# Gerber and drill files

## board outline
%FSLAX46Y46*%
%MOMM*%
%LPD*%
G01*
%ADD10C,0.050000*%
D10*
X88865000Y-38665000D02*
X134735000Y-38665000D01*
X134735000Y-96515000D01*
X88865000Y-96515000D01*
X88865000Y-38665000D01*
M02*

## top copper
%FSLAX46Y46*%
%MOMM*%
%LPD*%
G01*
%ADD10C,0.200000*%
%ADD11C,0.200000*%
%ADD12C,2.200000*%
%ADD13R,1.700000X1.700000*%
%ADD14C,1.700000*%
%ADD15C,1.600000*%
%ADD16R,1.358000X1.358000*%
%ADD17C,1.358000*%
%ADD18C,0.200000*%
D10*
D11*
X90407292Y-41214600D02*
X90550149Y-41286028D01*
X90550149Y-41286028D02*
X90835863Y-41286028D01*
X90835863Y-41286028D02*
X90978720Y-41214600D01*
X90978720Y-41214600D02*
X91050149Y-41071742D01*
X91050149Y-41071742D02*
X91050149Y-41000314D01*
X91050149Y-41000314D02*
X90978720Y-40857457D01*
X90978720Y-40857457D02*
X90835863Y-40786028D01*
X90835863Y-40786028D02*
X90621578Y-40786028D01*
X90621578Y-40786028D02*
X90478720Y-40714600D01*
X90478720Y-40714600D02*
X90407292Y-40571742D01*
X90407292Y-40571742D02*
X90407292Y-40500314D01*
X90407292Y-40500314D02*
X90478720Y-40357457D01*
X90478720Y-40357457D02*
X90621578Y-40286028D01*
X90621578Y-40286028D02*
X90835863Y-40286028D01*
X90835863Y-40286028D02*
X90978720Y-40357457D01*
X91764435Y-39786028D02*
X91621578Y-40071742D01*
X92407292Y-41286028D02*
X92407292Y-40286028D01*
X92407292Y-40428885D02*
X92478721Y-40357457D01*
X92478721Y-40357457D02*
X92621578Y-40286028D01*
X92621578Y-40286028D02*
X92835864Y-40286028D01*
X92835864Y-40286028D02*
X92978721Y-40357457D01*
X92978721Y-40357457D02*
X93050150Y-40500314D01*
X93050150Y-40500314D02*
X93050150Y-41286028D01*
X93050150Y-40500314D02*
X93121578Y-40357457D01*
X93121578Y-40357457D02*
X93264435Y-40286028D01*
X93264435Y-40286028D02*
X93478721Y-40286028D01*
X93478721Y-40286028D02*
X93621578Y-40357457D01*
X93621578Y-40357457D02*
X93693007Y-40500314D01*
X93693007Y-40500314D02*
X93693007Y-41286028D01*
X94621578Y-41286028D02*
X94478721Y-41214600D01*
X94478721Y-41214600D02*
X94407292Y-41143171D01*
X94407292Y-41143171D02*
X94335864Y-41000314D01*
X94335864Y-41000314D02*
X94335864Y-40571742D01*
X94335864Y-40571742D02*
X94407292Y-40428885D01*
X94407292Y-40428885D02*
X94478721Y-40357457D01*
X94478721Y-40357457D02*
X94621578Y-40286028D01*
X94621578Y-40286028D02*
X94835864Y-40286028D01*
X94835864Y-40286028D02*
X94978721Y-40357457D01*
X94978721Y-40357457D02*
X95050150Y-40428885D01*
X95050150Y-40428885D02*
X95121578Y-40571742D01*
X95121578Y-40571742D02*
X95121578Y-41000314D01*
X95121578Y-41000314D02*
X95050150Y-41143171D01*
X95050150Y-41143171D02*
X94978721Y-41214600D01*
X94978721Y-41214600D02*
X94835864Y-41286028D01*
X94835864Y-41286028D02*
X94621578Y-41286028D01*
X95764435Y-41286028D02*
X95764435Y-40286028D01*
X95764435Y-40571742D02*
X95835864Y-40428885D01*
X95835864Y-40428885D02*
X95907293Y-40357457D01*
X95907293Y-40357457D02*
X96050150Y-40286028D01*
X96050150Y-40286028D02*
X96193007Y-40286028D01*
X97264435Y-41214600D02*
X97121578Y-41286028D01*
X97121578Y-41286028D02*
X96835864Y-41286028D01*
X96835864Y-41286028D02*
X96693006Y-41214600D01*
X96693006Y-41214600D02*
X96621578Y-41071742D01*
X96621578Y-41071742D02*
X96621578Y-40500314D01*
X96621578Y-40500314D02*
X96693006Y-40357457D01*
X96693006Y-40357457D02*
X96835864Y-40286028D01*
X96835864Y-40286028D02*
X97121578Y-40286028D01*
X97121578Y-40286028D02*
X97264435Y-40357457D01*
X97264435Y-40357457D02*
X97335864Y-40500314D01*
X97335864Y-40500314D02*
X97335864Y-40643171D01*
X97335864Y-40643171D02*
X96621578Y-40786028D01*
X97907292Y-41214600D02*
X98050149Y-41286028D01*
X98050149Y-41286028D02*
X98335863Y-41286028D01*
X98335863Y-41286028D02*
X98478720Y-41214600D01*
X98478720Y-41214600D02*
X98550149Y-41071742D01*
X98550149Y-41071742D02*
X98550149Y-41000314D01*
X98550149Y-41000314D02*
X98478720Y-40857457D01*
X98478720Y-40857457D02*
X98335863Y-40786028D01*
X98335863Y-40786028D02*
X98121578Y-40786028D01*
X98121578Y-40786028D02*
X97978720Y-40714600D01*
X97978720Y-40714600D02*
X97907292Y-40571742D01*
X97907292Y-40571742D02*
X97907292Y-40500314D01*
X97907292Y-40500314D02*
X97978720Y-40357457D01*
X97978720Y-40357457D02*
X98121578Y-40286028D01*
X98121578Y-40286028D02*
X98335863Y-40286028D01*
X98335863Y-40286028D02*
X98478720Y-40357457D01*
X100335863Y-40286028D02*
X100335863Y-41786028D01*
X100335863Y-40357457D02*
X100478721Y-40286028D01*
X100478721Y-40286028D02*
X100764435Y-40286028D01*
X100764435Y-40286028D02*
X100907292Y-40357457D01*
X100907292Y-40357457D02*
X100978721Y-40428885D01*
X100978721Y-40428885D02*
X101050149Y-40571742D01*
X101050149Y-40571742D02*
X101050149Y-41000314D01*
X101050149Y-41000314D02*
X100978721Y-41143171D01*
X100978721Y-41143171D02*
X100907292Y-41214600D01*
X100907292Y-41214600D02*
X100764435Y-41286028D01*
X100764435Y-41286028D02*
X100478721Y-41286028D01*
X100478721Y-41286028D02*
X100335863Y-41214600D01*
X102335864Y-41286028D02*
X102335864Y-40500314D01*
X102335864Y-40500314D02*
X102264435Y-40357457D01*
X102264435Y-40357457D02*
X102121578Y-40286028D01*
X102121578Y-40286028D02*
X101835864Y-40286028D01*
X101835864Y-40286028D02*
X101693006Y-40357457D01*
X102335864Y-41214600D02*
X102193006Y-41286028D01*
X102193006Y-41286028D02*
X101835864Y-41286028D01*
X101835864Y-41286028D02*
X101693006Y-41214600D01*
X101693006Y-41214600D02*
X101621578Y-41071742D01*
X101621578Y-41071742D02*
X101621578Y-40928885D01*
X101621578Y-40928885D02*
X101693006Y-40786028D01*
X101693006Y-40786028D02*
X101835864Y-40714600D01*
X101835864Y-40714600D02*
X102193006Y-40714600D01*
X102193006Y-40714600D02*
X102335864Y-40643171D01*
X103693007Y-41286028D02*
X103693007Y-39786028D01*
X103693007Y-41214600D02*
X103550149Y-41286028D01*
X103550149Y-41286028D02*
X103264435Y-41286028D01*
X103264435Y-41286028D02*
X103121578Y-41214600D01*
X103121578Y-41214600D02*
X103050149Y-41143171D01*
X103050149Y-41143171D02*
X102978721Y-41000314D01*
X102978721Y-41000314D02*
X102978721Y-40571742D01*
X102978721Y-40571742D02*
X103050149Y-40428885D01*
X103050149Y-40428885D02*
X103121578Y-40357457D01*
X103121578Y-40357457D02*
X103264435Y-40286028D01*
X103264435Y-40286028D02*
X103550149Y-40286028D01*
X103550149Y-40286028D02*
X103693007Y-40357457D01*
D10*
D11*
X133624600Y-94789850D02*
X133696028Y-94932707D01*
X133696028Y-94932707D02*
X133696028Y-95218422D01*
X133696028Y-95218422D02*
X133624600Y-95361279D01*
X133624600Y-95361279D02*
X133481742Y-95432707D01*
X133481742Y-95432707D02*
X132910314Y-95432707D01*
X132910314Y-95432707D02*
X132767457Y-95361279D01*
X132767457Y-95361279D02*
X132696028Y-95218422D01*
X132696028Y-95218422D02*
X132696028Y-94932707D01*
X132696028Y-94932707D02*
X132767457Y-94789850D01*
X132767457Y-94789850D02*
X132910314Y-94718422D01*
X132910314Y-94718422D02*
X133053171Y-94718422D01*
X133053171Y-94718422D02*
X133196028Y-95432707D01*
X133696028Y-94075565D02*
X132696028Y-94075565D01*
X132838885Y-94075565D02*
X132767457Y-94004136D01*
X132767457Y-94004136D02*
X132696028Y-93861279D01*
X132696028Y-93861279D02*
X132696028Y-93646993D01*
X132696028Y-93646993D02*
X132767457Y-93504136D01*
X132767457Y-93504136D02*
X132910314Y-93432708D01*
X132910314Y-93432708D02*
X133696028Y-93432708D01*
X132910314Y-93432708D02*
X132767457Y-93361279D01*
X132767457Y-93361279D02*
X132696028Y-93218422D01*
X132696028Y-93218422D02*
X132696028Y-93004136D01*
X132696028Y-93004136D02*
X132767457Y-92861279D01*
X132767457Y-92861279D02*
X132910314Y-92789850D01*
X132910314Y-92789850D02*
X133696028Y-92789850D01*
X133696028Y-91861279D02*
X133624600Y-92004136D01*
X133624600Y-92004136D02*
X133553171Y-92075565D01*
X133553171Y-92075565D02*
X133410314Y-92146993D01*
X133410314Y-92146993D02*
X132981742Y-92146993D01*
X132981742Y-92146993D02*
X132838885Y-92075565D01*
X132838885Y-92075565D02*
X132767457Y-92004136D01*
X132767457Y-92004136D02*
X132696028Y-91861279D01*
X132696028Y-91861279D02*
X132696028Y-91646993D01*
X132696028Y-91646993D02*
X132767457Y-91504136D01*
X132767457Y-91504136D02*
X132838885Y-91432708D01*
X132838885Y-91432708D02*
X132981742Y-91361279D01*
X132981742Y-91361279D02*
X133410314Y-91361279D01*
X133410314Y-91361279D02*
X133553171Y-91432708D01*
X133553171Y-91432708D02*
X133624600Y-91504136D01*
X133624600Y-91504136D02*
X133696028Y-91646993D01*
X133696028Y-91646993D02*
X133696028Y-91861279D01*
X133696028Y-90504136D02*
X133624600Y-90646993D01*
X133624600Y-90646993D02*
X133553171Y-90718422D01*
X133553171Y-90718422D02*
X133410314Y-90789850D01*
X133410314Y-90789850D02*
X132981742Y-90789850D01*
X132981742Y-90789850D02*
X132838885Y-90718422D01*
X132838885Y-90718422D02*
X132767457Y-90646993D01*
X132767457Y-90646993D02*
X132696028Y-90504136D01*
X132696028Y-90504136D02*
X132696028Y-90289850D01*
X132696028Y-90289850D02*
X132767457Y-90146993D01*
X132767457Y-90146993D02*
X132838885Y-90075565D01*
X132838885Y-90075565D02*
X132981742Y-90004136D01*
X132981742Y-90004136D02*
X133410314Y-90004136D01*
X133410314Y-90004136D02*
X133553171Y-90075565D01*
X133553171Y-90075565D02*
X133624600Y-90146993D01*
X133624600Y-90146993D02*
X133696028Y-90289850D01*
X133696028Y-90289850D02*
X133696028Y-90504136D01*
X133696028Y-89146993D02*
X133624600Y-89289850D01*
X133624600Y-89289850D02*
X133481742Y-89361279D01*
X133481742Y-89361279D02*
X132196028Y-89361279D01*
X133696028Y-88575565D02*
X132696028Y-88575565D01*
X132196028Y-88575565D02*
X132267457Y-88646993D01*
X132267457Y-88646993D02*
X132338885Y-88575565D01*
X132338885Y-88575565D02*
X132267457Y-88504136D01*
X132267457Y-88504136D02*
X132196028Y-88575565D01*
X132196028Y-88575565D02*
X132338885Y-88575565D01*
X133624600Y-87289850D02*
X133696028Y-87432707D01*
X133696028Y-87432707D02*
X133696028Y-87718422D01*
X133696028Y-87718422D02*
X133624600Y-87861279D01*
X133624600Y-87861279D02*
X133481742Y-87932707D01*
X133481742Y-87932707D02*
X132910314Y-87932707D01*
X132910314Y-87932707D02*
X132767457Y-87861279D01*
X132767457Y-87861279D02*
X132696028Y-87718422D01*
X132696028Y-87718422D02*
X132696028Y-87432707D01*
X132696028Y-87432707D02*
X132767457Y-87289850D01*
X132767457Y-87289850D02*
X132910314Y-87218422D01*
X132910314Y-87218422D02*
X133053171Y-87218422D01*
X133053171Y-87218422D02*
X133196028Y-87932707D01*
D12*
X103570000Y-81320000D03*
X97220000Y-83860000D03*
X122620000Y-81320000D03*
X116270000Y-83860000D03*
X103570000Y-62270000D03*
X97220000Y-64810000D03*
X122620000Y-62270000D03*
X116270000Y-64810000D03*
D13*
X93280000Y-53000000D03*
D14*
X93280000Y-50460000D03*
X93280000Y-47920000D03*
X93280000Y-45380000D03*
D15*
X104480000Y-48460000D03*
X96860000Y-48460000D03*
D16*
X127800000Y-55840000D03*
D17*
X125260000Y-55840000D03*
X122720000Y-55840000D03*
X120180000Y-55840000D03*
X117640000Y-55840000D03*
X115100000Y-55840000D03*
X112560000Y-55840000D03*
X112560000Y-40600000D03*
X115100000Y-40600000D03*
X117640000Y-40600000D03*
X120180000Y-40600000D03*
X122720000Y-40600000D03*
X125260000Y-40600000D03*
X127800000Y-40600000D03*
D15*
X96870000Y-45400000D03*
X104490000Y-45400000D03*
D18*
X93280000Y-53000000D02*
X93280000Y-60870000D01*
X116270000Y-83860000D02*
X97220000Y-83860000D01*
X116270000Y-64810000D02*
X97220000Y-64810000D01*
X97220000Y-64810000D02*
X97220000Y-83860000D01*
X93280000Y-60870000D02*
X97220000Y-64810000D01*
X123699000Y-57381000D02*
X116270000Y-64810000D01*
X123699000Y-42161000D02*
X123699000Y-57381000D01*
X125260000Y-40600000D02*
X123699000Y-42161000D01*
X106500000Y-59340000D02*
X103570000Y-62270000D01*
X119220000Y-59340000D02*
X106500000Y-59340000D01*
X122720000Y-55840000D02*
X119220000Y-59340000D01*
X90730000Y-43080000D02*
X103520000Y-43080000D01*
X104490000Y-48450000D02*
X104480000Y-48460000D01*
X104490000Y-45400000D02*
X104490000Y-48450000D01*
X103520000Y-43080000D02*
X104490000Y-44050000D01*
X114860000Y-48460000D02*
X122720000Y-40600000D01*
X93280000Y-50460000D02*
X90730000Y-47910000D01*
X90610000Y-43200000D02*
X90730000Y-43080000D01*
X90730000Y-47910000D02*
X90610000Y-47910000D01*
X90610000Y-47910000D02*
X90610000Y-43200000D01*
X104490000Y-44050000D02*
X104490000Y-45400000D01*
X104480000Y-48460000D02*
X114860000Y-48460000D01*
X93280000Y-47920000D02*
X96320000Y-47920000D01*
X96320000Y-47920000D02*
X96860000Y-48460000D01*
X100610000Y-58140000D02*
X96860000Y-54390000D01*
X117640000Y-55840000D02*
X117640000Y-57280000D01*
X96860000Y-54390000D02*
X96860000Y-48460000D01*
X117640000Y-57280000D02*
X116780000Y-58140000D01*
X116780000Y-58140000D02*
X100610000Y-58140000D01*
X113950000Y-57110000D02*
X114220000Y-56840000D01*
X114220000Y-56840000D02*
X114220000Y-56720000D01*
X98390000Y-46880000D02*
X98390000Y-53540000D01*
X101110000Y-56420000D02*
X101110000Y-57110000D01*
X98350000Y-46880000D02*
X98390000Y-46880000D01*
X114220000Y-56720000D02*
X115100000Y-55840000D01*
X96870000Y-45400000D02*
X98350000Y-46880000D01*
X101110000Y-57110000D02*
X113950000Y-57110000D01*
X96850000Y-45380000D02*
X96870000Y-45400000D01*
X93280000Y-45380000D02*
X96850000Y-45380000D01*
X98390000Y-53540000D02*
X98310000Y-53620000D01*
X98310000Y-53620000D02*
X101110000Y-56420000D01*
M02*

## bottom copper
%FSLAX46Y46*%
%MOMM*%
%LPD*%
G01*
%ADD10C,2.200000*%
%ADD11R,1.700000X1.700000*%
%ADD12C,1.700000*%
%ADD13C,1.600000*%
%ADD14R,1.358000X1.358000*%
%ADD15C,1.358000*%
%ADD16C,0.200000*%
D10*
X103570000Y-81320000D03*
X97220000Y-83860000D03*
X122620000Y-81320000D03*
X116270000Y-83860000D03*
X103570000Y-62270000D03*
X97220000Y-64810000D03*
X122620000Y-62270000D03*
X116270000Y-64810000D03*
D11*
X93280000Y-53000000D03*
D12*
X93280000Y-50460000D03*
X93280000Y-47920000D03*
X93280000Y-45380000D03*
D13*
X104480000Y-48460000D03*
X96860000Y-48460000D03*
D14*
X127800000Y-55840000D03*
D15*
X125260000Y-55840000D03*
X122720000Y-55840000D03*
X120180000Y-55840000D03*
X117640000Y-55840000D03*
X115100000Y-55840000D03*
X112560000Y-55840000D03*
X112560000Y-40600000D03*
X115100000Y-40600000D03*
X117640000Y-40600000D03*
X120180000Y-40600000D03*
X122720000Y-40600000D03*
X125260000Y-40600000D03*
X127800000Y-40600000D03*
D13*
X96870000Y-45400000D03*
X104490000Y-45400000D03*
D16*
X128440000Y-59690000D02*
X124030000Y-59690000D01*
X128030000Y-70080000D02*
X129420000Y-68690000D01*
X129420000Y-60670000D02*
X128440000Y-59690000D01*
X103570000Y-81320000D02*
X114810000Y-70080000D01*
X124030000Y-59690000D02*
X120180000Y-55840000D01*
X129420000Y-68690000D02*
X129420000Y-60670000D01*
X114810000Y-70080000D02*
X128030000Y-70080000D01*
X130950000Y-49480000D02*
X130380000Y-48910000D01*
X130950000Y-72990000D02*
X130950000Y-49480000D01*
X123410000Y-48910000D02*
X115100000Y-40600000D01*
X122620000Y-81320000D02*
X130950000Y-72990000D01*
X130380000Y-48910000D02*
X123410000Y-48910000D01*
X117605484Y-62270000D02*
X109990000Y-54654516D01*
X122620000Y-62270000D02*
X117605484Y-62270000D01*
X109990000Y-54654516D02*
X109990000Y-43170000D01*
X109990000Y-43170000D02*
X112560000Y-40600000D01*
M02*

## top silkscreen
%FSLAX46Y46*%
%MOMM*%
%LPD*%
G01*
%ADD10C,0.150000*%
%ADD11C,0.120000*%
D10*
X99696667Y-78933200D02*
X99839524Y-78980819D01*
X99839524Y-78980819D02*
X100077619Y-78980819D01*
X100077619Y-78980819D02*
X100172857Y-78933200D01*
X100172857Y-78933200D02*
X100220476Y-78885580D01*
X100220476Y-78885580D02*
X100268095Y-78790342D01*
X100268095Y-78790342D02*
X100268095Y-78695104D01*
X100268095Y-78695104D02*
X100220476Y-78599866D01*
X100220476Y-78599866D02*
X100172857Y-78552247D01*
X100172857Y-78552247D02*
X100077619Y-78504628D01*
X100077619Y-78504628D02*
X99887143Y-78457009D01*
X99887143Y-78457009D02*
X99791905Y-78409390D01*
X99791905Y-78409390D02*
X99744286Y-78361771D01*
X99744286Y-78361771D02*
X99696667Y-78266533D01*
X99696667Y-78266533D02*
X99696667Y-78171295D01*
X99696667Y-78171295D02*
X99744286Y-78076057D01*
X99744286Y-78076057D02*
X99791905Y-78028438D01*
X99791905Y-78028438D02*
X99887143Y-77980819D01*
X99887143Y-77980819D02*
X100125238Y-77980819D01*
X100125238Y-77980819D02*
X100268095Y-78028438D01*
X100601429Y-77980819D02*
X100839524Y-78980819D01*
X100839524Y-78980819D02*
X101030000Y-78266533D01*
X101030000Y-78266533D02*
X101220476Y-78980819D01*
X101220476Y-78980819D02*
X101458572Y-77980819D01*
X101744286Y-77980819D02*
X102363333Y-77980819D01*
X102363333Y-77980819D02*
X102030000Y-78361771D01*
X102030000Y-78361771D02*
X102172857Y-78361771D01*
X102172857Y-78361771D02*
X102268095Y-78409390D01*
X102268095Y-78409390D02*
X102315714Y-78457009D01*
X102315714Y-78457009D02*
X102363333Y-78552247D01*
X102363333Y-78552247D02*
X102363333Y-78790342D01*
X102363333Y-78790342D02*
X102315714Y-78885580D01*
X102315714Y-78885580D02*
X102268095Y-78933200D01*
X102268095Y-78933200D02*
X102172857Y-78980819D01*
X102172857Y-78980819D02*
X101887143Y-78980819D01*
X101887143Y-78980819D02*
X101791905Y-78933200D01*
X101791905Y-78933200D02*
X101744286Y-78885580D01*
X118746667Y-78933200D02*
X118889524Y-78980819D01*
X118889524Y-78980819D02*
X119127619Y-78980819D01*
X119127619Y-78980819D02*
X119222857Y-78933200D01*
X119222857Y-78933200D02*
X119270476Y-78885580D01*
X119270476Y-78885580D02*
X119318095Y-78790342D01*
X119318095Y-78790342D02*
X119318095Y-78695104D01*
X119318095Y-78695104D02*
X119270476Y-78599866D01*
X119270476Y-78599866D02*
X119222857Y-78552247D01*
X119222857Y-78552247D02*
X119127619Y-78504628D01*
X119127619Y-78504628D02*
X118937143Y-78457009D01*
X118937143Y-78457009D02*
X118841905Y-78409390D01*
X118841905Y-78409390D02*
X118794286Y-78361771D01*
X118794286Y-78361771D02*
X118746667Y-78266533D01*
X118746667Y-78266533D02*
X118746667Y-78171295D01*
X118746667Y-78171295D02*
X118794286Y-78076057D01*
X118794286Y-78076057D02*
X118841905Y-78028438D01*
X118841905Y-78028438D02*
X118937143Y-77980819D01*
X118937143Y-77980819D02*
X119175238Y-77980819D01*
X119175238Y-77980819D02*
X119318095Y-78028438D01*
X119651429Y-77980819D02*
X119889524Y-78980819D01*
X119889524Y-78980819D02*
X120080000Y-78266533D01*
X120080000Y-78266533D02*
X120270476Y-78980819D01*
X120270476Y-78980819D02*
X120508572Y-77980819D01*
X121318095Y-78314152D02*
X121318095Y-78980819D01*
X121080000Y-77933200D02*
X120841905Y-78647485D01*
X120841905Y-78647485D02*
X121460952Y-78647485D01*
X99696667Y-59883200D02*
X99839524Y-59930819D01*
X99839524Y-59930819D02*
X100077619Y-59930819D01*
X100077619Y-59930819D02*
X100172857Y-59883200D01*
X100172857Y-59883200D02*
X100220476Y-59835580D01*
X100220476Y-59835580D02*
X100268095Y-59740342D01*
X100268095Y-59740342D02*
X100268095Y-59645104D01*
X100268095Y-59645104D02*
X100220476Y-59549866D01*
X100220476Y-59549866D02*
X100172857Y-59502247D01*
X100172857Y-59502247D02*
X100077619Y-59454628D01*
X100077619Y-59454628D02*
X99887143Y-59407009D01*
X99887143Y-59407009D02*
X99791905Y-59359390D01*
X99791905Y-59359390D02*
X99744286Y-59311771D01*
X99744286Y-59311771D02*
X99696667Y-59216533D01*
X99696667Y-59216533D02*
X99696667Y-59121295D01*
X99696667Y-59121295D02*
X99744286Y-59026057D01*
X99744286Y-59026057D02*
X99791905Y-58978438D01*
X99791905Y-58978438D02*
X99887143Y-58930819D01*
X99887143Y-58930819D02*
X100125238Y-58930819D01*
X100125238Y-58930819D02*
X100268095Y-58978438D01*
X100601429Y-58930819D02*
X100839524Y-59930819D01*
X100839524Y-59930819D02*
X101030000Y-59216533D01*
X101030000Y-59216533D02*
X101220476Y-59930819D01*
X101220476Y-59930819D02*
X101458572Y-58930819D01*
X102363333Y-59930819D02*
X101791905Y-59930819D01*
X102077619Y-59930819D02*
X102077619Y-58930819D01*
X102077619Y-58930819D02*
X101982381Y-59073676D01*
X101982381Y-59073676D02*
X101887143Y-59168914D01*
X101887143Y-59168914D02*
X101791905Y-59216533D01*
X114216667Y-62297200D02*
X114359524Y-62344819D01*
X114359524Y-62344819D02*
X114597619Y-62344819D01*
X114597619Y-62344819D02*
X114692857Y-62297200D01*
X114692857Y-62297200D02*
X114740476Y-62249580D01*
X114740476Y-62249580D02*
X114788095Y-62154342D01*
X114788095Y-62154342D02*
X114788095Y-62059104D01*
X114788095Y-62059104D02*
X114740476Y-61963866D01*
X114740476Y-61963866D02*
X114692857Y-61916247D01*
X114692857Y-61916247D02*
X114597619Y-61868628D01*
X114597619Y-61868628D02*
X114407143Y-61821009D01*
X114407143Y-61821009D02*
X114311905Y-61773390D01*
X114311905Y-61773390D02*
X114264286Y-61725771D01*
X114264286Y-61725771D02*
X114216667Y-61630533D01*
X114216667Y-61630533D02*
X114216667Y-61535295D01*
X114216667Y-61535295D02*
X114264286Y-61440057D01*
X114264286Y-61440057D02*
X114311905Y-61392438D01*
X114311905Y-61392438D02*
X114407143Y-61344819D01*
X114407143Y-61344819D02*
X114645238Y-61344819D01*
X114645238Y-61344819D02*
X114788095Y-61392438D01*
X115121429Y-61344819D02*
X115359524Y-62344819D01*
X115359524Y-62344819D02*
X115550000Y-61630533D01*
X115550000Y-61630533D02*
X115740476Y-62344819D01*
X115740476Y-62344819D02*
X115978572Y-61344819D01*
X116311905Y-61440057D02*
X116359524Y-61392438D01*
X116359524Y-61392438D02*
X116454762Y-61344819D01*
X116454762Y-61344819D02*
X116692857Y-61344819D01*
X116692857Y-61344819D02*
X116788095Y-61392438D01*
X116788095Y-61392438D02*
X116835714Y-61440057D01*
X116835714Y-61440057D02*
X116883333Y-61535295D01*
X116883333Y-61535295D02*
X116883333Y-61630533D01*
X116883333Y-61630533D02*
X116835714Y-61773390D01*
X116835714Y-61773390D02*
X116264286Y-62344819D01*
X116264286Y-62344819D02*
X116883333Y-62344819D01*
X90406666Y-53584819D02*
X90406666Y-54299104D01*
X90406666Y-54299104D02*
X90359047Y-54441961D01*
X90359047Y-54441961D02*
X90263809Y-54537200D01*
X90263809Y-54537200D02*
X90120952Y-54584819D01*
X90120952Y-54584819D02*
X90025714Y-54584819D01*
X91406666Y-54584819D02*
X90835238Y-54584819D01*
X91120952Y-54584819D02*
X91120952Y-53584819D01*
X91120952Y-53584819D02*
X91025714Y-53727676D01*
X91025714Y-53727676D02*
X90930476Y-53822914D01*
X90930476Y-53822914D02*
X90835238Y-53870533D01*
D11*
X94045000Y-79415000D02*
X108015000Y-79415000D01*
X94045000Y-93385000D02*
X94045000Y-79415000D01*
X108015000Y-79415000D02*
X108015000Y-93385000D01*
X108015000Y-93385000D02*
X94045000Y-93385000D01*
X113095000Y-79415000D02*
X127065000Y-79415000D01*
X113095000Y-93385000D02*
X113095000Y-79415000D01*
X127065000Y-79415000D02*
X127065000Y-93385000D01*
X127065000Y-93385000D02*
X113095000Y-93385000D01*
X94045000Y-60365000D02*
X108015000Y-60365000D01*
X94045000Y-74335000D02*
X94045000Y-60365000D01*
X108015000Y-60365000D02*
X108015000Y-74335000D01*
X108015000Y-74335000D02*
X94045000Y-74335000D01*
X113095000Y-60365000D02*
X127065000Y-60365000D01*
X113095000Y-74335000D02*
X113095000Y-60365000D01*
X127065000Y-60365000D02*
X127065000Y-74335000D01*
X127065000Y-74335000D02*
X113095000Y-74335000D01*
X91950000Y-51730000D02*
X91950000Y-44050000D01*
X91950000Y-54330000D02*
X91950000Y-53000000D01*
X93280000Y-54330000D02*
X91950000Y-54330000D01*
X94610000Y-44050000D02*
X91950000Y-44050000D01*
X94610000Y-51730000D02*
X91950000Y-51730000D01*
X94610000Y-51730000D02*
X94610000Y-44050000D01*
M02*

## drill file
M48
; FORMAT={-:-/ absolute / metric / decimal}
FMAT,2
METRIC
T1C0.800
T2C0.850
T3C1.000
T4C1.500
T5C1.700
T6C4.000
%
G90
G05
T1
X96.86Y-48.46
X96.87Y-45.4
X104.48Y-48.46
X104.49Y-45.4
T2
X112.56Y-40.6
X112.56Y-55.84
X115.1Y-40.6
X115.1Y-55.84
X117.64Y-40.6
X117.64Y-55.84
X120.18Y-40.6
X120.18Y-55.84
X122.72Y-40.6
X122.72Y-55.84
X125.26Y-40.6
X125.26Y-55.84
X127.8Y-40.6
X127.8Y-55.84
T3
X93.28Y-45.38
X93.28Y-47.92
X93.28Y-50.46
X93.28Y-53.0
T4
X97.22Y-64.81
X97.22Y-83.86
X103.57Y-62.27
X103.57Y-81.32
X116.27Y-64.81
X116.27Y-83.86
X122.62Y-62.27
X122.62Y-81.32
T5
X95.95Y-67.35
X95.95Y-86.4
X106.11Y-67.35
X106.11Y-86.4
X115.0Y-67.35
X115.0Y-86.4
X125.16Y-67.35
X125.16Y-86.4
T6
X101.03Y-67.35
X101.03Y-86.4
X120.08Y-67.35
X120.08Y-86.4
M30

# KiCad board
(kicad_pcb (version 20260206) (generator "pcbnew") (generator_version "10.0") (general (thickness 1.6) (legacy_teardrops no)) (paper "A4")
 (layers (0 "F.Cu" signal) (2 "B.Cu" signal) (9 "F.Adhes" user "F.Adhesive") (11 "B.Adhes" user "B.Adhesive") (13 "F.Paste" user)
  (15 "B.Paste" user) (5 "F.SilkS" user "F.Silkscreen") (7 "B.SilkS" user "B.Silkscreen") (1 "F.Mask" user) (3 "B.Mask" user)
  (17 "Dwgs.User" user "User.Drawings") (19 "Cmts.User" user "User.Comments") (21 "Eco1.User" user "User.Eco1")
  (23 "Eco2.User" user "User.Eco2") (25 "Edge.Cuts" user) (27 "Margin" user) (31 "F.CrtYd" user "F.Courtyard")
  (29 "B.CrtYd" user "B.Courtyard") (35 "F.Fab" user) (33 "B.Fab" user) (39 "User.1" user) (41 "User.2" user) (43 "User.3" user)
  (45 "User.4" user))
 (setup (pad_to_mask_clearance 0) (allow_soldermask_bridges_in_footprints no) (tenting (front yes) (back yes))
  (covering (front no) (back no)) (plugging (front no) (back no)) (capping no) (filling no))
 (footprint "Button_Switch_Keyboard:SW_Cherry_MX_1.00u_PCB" (layer "F.Cu") (at 103.57 81.32)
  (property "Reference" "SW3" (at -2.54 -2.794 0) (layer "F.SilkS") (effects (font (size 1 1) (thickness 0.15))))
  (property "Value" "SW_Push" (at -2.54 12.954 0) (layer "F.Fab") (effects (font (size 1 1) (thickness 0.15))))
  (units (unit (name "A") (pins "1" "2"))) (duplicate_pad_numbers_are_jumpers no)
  (fp_line (start -9.525 -1.905) (end 4.445 -1.905) (stroke (width 0.12) (type solid)) (layer "F.SilkS"))
  (fp_line (start -9.525 12.065) (end -9.525 -1.905) (stroke (width 0.12) (type solid)) (layer "F.SilkS"))
  (fp_line (start 4.445 -1.905) (end 4.445 12.065) (stroke (width 0.12) (type solid)) (layer "F.SilkS"))
  (fp_line (start 4.445 12.065) (end -9.525 12.065) (stroke (width 0.12) (type solid)) (layer "F.SilkS"))
  (pad "" np_thru_hole circle (at -7.62 5.08) (size 1.7 1.7) (drill 1.7) (layers "*.Cu" "*.Mask"))
  (pad "" np_thru_hole circle (at -2.54 5.08) (size 4 4) (drill 4) (layers "*.Cu" "*.Mask"))
  (pad "" np_thru_hole circle (at 2.54 5.08) (size 1.7 1.7) (drill 1.7) (layers "*.Cu" "*.Mask"))
  (pad "1" thru_hole circle (at 0 0) (size 2.2 2.2) (drill 1.5) (layers "*.Cu" "*.Mask") (remove_unused_layers no) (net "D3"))
  (pad "2" thru_hole circle (at -6.35 2.54) (size 2.2 2.2) (drill 1.5) (layers "*.Cu" "*.Mask") (remove_unused_layers no) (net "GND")))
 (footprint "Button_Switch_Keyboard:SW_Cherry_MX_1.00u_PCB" (layer "F.Cu") (at 122.62 81.32)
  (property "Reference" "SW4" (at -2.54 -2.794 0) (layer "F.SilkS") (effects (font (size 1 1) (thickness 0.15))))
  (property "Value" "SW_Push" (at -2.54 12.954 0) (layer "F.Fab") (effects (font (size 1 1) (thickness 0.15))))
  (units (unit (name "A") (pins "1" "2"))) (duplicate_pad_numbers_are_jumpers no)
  (fp_line (start -9.525 -1.905) (end 4.445 -1.905) (stroke (width 0.12) (type solid)) (layer "F.SilkS"))
  (fp_line (start -9.525 12.065) (end -9.525 -1.905) (stroke (width 0.12) (type solid)) (layer "F.SilkS"))
  (fp_line (start 4.445 -1.905) (end 4.445 12.065) (stroke (width 0.12) (type solid)) (layer "F.SilkS"))
  (fp_line (start 4.445 12.065) (end -9.525 12.065) (stroke (width 0.12) (type solid)) (layer "F.SilkS"))
  (pad "" np_thru_hole circle (at -7.62 5.08) (size 1.7 1.7) (drill 1.7) (layers "*.Cu" "*.Mask"))
  (pad "" np_thru_hole circle (at -2.54 5.08) (size 4 4) (drill 4) (layers "*.Cu" "*.Mask"))
  (pad "" np_thru_hole circle (at 2.54 5.08) (size 1.7 1.7) (drill 1.7) (layers "*.Cu" "*.Mask"))
  (pad "1" thru_hole circle (at 0 0) (size 2.2 2.2) (drill 1.5) (layers "*.Cu" "*.Mask") (remove_unused_layers no) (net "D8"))
  (pad "2" thru_hole circle (at -6.35 2.54) (size 2.2 2.2) (drill 1.5) (layers "*.Cu" "*.Mask") (remove_unused_layers no) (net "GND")))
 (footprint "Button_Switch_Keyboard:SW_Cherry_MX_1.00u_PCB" (layer "F.Cu") (at 103.57 62.27)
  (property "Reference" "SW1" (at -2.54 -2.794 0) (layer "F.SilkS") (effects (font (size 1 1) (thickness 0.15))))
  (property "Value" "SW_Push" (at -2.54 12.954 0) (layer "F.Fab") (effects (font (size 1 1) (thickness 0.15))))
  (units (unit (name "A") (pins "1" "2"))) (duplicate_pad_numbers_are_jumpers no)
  (fp_line (start -9.525 -1.905) (end 4.445 -1.905) (stroke (width 0.12) (type solid)) (layer "F.SilkS"))
  (fp_line (start -9.525 12.065) (end -9.525 -1.905) (stroke (width 0.12) (type solid)) (layer "F.SilkS"))
  (fp_line (start 4.445 -1.905) (end 4.445 12.065) (stroke (width 0.12) (type solid)) (layer "F.SilkS"))
  (fp_line (start 4.445 12.065) (end -9.525 12.065) (stroke (width 0.12) (type solid)) (layer "F.SilkS"))
  (pad "" np_thru_hole circle (at -7.62 5.08) (size 1.7 1.7) (drill 1.7) (layers "*.Cu" "*.Mask"))
  (pad "" np_thru_hole circle (at -2.54 5.08) (size 4 4) (drill 4) (layers "*.Cu" "*.Mask"))
  (pad "" np_thru_hole circle (at 2.54 5.08) (size 1.7 1.7) (drill 1.7) (layers "*.Cu" "*.Mask"))
  (pad "1" thru_hole circle (at 0 0) (size 2.2 2.2) (drill 1.5) (layers "*.Cu" "*.Mask") (remove_unused_layers no) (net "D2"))
  (pad "2" thru_hole circle (at -6.35 2.54) (size 2.2 2.2) (drill 1.5) (layers "*.Cu" "*.Mask") (remove_unused_layers no) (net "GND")))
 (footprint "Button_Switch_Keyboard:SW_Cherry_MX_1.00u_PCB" (layer "F.Cu") (at 122.62 62.27)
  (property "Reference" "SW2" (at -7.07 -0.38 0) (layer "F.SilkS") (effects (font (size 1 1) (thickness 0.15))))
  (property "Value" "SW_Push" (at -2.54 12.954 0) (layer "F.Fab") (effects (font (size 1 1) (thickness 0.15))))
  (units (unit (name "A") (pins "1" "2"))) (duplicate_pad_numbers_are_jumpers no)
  (fp_line (start -9.525 -1.905) (end 4.445 -1.905) (stroke (width 0.12) (type solid)) (layer "F.SilkS"))
  (fp_line (start -9.525 12.065) (end -9.525 -1.905) (stroke (width 0.12) (type solid)) (layer "F.SilkS"))
  (fp_line (start 4.445 -1.905) (end 4.445 12.065) (stroke (width 0.12) (type solid)) (layer "F.SilkS"))
  (fp_line (start 4.445 12.065) (end -9.525 12.065) (stroke (width 0.12) (type solid)) (layer "F.SilkS"))
  (pad "" np_thru_hole circle (at -7.62 5.08) (size 1.7 1.7) (drill 1.7) (layers "*.Cu" "*.Mask"))
  (pad "" np_thru_hole circle (at -2.54 5.08) (size 4 4) (drill 4) (layers "*.Cu" "*.Mask"))
  (pad "" np_thru_hole circle (at 2.54 5.08) (size 1.7 1.7) (drill 1.7) (layers "*.Cu" "*.Mask"))
  (pad "1" thru_hole circle (at 0 0) (size 2.2 2.2) (drill 1.5) (layers "*.Cu" "*.Mask") (remove_unused_layers no) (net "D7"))
  (pad "2" thru_hole circle (at -6.35 2.54) (size 2.2 2.2) (drill 1.5) (layers "*.Cu" "*.Mask") (remove_unused_layers no) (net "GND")))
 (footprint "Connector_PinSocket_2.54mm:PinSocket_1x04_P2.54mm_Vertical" (layer "F.Cu") (at 93.28 53 180)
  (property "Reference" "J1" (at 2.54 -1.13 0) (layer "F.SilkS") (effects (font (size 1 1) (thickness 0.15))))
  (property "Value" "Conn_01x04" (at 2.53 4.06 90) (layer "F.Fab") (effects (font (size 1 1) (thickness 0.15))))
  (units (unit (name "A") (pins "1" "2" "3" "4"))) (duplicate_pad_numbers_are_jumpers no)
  (fp_line (start 1.33 1.27) (end 1.33 8.95) (stroke (width 0.12) (type solid)) (layer "F.SilkS"))
  (fp_line (start 1.33 -1.33) (end 1.33 0) (stroke (width 0.12) (type solid)) (layer "F.SilkS"))
  (fp_line (start 0 -1.33) (end 1.33 -1.33) (stroke (width 0.12) (type solid)) (layer "F.SilkS"))
  (fp_line (start -1.33 8.95) (end 1.33 8.95) (stroke (width 0.12) (type solid)) (layer "F.SilkS"))
  (fp_line (start -1.33 1.27) (end 1.33 1.27) (stroke (width 0.12) (type solid)) (layer "F.SilkS"))
  (fp_line (start -1.33 1.27) (end -1.33 8.95) (stroke (width 0.12) (type solid)) (layer "F.SilkS"))
  (pad "1" thru_hole rect (at 0 0 180) (size 1.7 1.7) (drill 1) (layers "*.Cu" "*.Mask") (remove_unused_layers no) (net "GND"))
  (pad "2" thru_hole circle (at 0 2.54 180) (size 1.7 1.7) (drill 1) (layers "*.Cu" "*.Mask") (remove_unused_layers no) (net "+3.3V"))
  (pad "3" thru_hole circle (at 0 5.08 180) (size 1.7 1.7) (drill 1) (layers "*.Cu" "*.Mask") (remove_unused_layers no) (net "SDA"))
  (pad "4" thru_hole circle (at 0 7.62 180) (size 1.7 1.7) (drill 1) (layers "*.Cu" "*.Mask") (remove_unused_layers no) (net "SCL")))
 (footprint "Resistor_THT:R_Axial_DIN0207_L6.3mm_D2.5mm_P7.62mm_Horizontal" (layer "B.Cu") (at 104.48 48.46 180)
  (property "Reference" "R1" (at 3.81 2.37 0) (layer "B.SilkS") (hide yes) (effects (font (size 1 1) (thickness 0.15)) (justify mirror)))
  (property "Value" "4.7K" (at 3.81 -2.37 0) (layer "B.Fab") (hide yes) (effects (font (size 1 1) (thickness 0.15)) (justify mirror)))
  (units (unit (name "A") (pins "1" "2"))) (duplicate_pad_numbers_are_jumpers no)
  (pad "1" thru_hole circle (at 0 0 180) (size 1.6 1.6) (drill 0.8) (layers "*.Cu" "*.Mask") (remove_unused_layers no) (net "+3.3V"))
  (pad "2" thru_hole circle (at 7.62 0 180) (size 1.6 1.6) (drill 0.8) (layers "*.Cu" "*.Mask") (remove_unused_layers no) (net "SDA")))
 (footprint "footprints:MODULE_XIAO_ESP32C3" (layer "B.Cu") (at 120.2435 48.22 90)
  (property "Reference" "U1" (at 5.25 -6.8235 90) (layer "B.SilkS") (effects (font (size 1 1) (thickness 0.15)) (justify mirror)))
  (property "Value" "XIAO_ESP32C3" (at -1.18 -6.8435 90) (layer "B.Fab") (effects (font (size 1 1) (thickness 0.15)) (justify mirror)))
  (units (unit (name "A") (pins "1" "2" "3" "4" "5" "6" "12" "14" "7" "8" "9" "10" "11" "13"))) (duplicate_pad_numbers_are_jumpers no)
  (pad "1" thru_hole rect (at -7.62 7.5565 90) (size 1.358 1.358) (drill 0.85) (layers "*.Cu" "*.Mask") (remove_unused_layers no)
   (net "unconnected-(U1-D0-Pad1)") (solder_mask_margin 0.102))
  (pad "2" thru_hole circle (at -7.62 5.0165 90) (size 1.358 1.358) (drill 0.85) (layers "*.Cu" "*.Mask") (remove_unused_layers no)
   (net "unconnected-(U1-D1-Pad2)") (solder_mask_margin 0.102))
  (pad "3" thru_hole circle (at -7.62 2.4765 90) (size 1.358 1.358) (drill 0.85) (layers "*.Cu" "*.Mask") (remove_unused_layers no)
   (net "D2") (solder_mask_margin 0.102))
  (pad "4" thru_hole circle (at -7.62 -0.0635 90) (size 1.358 1.358) (drill 0.85) (layers "*.Cu" "*.Mask") (remove_unused_layers no)
   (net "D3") (solder_mask_margin 0.102))
  (pad "5" thru_hole circle (at -7.62 -2.6035 90) (size 1.358 1.358) (drill 0.85) (layers "*.Cu" "*.Mask") (remove_unused_layers no)
   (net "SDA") (solder_mask_margin 0.102))
  (pad "6" thru_hole circle (at -7.62 -5.1435 90) (size 1.358 1.358) (drill 0.85) (layers "*.Cu" "*.Mask") (remove_unused_layers no)
   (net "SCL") (solder_mask_margin 0.102))
  (pad "7" thru_hole circle (at -7.62 -7.6835 90) (size 1.358 1.358) (drill 0.85) (layers "*.Cu" "*.Mask") (remove_unused_layers no)
   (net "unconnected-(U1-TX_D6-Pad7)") (solder_mask_margin 0.102))
  (pad "8" thru_hole circle (at 7.62 -7.6835 90) (size 1.358 1.358) (drill 0.85) (layers "*.Cu" "*.Mask") (remove_unused_layers no)
   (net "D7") (solder_mask_margin 0.102))
  (pad "9" thru_hole circle (at 7.62 -5.1435 90) (size 1.358 1.358) (drill 0.85) (layers "*.Cu" "*.Mask") (remove_unused_layers no)
   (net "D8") (solder_mask_margin 0.102))
  (pad "10" thru_hole circle (at 7.62 -2.6035 90) (size 1.358 1.358) (drill 0.85) (layers "*.Cu" "*.Mask") (remove_unused_layers no)
   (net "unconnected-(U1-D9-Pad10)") (solder_mask_margin 0.102))
  (pad "11" thru_hole circle (at 7.62 -0.0635 90) (size 1.358 1.358) (drill 0.85) (layers "*.Cu" "*.Mask") (remove_unused_layers no)
   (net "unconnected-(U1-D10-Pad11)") (solder_mask_margin 0.102))
  (pad "12" thru_hole circle (at 7.62 2.4765 90) (size 1.358 1.358) (drill 0.85) (layers "*.Cu" "*.Mask") (remove_unused_layers no)
   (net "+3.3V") (solder_mask_margin 0.102))
  (pad "13" thru_hole circle (at 7.62 5.0165 90) (size 1.358 1.358) (drill 0.85) (layers "*.Cu" "*.Mask") (remove_unused_layers no)
   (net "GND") (solder_mask_margin 0.102))
  (pad "14" thru_hole circle (at 7.62 7.5565 90) (size 1.358 1.358) (drill 0.85) (layers "*.Cu" "*.Mask") (remove_unused_layers no)
   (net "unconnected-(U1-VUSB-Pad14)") (solder_mask_margin 0.102)))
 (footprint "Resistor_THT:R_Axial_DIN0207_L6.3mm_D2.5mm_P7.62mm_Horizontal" (layer "B.Cu") (at 96.87 45.4)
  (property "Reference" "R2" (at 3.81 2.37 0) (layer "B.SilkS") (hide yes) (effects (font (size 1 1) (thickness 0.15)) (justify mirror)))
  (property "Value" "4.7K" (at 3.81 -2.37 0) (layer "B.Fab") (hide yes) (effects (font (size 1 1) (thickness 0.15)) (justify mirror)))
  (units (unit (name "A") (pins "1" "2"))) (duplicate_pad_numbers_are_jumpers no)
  (pad "1" thru_hole circle (at 0 0) (size 1.6 1.6) (drill 0.8) (layers "*.Cu" "*.Mask") (remove_unused_layers no) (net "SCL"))
  (pad "2" thru_hole circle (at 7.62 0) (size 1.6 1.6) (drill 0.8) (layers "*.Cu" "*.Mask") (remove_unused_layers no) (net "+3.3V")))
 (gr_rect (start 88.865 38.665) (end 134.735 96.515) (stroke (width 0.05) (type default)) (fill no) (layer "Edge.Cuts"))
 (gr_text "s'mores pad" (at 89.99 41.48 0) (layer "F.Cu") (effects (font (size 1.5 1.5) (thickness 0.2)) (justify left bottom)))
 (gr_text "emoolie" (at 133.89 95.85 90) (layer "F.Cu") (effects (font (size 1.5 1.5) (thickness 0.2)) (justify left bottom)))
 (segment (start 128.44 59.69) (end 124.03 59.69) (width 0.2) (layer "B.Cu") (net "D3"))
 (segment (start 128.03 70.08) (end 129.42 68.69) (width 0.2) (layer "B.Cu") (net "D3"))
 (segment (start 129.42 60.67) (end 128.44 59.69) (width 0.2) (layer "B.Cu") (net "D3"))
 (segment (start 103.57 81.32) (end 114.81 70.08) (width 0.2) (layer "B.Cu") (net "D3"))
 (segment (start 124.03 59.69) (end 120.18 55.84) (width 0.2) (layer "B.Cu") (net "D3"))
 (segment (start 129.42 68.69) (end 129.42 60.67) (width 0.2) (layer "B.Cu") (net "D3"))
 (segment (start 114.81 70.08) (end 128.03 70.08) (width 0.2) (layer "B.Cu") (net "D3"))
 (segment (start 93.28 53) (end 93.28 60.87) (width 0.2) (layer "F.Cu") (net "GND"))
 (segment (start 116.27 83.86) (end 97.22 83.86) (width 0.2) (layer "F.Cu") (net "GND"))
 (segment (start 116.27 64.81) (end 97.22 64.81) (width 0.2) (layer "F.Cu") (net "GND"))
 (segment (start 97.22 64.81) (end 97.22 83.86) (width 0.2) (layer "F.Cu") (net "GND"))
 (segment (start 93.28 60.87) (end 97.22 64.81) (width 0.2) (layer "F.Cu") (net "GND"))
 (segment (start 123.699 57.381) (end 116.27 64.81) (width 0.2) (layer "F.Cu") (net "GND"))
 (segment (start 123.699 42.161) (end 123.699 57.381) (width 0.2) (layer "F.Cu") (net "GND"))
 (segment (start 125.26 40.6) (end 123.699 42.161) (width 0.2) (layer "F.Cu") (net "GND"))
 (segment (start 130.95 49.48) (end 130.38 48.91) (width 0.2) (layer "B.Cu") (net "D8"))
 (segment (start 130.95 72.99) (end 130.95 49.48) (width 0.2) (layer "B.Cu") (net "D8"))
 (segment (start 123.41 48.91) (end 115.1 40.6) (width 0.2) (layer "B.Cu") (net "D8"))
 (segment (start 122.62 81.32) (end 130.95 72.99) (width 0.2) (layer "B.Cu") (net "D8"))
 (segment (start 130.38 48.91) (end 123.41 48.91) (width 0.2) (layer "B.Cu") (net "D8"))
 (segment (start 106.5 59.34) (end 103.57 62.27) (width 0.2) (layer "F.Cu") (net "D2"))
 (segment (start 119.22 59.34) (end 106.5 59.34) (width 0.2) (layer "F.Cu") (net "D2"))
 (segment (start 122.72 55.84) (end 119.22 59.34) (width 0.2) (layer "F.Cu") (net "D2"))
 (segment (start 117.605484 62.27) (end 109.99 54.654516) (width 0.2) (layer "B.Cu") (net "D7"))
 (segment (start 122.62 62.27) (end 117.605484 62.27) (width 0.2) (layer "B.Cu") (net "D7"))
 (segment (start 109.99 54.654516) (end 109.99 43.17) (width 0.2) (layer "B.Cu") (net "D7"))
 (segment (start 109.99 43.17) (end 112.56 40.6) (width 0.2) (layer "B.Cu") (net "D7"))
 (segment (start 90.73 43.08) (end 103.52 43.08) (width 0.2) (layer "F.Cu") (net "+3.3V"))
 (segment (start 104.49 48.45) (end 104.48 48.46) (width 0.2) (layer "F.Cu") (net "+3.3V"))
 (segment (start 104.49 45.4) (end 104.49 48.45) (width 0.2) (layer "F.Cu") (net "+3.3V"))
 (segment (start 103.52 43.08) (end 104.49 44.05) (width 0.2) (layer "F.Cu") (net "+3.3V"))
 (segment (start 114.86 48.46) (end 122.72 40.6) (width 0.2) (layer "F.Cu") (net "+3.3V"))
 (segment (start 93.28 50.46) (end 90.73 47.91) (width 0.2) (layer "F.Cu") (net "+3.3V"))
 (segment (start 90.61 43.2) (end 90.73 43.08) (width 0.2) (layer "F.Cu") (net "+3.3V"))
 (segment (start 90.73 47.91) (end 90.61 47.91) (width 0.2) (layer "F.Cu") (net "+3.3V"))
 (segment (start 90.61 47.91) (end 90.61 43.2) (width 0.2) (layer "F.Cu") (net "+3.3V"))
 (segment (start 104.49 44.05) (end 104.49 45.4) (width 0.2) (layer "F.Cu") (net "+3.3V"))
 (segment (start 104.48 48.46) (end 114.86 48.46) (width 0.2) (layer "F.Cu") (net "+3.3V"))
 (segment (start 93.28 47.92) (end 96.32 47.92) (width 0.2) (layer "F.Cu") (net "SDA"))
 (segment (start 96.32 47.92) (end 96.86 48.46) (width 0.2) (layer "F.Cu") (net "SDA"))
 (segment (start 100.61 58.14) (end 96.86 54.39) (width 0.2) (layer "F.Cu") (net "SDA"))
 (segment (start 117.64 55.84) (end 117.64 57.28) (width 0.2) (layer "F.Cu") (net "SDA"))
 (segment (start 96.86 54.39) (end 96.86 48.46) (width 0.2) (layer "F.Cu") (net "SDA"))
 (segment (start 117.64 57.28) (end 116.78 58.14) (width 0.2) (layer "F.Cu") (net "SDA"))
 (segment (start 116.78 58.14) (end 100.61 58.14) (width 0.2) (layer "F.Cu") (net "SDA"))
 (segment (start 113.95 57.11) (end 114.22 56.84) (width 0.2) (layer "F.Cu") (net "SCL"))
 (segment (start 114.22 56.84) (end 114.22 56.72) (width 0.2) (layer "F.Cu") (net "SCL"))
 (segment (start 98.39 46.88) (end 98.39 53.54) (width 0.2) (layer "F.Cu") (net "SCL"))
 (segment (start 101.11 56.42) (end 101.11 57.11) (width 0.2) (layer "F.Cu") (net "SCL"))
 (segment (start 98.35 46.88) (end 98.39 46.88) (width 0.2) (layer "F.Cu") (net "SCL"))
 (segment (start 114.22 56.72) (end 115.1 55.84) (width 0.2) (layer "F.Cu") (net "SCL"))
 (segment (start 96.87 45.4) (end 98.35 46.88) (width 0.2) (layer "F.Cu") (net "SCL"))
 (segment (start 101.11 57.11) (end 113.95 57.11) (width 0.2) (layer "F.Cu") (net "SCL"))
 (segment (start 96.85 45.38) (end 96.87 45.4) (width 0.2) (layer "F.Cu") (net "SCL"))
 (segment (start 93.28 45.38) (end 96.85 45.38) (width 0.2) (layer "F.Cu") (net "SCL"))
 (segment (start 98.39 53.54) (end 98.31 53.62) (width 0.2) (layer "F.Cu") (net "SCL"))
 (segment (start 98.31 53.62) (end 101.11 56.42) (width 0.2) (layer "F.Cu") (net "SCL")))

